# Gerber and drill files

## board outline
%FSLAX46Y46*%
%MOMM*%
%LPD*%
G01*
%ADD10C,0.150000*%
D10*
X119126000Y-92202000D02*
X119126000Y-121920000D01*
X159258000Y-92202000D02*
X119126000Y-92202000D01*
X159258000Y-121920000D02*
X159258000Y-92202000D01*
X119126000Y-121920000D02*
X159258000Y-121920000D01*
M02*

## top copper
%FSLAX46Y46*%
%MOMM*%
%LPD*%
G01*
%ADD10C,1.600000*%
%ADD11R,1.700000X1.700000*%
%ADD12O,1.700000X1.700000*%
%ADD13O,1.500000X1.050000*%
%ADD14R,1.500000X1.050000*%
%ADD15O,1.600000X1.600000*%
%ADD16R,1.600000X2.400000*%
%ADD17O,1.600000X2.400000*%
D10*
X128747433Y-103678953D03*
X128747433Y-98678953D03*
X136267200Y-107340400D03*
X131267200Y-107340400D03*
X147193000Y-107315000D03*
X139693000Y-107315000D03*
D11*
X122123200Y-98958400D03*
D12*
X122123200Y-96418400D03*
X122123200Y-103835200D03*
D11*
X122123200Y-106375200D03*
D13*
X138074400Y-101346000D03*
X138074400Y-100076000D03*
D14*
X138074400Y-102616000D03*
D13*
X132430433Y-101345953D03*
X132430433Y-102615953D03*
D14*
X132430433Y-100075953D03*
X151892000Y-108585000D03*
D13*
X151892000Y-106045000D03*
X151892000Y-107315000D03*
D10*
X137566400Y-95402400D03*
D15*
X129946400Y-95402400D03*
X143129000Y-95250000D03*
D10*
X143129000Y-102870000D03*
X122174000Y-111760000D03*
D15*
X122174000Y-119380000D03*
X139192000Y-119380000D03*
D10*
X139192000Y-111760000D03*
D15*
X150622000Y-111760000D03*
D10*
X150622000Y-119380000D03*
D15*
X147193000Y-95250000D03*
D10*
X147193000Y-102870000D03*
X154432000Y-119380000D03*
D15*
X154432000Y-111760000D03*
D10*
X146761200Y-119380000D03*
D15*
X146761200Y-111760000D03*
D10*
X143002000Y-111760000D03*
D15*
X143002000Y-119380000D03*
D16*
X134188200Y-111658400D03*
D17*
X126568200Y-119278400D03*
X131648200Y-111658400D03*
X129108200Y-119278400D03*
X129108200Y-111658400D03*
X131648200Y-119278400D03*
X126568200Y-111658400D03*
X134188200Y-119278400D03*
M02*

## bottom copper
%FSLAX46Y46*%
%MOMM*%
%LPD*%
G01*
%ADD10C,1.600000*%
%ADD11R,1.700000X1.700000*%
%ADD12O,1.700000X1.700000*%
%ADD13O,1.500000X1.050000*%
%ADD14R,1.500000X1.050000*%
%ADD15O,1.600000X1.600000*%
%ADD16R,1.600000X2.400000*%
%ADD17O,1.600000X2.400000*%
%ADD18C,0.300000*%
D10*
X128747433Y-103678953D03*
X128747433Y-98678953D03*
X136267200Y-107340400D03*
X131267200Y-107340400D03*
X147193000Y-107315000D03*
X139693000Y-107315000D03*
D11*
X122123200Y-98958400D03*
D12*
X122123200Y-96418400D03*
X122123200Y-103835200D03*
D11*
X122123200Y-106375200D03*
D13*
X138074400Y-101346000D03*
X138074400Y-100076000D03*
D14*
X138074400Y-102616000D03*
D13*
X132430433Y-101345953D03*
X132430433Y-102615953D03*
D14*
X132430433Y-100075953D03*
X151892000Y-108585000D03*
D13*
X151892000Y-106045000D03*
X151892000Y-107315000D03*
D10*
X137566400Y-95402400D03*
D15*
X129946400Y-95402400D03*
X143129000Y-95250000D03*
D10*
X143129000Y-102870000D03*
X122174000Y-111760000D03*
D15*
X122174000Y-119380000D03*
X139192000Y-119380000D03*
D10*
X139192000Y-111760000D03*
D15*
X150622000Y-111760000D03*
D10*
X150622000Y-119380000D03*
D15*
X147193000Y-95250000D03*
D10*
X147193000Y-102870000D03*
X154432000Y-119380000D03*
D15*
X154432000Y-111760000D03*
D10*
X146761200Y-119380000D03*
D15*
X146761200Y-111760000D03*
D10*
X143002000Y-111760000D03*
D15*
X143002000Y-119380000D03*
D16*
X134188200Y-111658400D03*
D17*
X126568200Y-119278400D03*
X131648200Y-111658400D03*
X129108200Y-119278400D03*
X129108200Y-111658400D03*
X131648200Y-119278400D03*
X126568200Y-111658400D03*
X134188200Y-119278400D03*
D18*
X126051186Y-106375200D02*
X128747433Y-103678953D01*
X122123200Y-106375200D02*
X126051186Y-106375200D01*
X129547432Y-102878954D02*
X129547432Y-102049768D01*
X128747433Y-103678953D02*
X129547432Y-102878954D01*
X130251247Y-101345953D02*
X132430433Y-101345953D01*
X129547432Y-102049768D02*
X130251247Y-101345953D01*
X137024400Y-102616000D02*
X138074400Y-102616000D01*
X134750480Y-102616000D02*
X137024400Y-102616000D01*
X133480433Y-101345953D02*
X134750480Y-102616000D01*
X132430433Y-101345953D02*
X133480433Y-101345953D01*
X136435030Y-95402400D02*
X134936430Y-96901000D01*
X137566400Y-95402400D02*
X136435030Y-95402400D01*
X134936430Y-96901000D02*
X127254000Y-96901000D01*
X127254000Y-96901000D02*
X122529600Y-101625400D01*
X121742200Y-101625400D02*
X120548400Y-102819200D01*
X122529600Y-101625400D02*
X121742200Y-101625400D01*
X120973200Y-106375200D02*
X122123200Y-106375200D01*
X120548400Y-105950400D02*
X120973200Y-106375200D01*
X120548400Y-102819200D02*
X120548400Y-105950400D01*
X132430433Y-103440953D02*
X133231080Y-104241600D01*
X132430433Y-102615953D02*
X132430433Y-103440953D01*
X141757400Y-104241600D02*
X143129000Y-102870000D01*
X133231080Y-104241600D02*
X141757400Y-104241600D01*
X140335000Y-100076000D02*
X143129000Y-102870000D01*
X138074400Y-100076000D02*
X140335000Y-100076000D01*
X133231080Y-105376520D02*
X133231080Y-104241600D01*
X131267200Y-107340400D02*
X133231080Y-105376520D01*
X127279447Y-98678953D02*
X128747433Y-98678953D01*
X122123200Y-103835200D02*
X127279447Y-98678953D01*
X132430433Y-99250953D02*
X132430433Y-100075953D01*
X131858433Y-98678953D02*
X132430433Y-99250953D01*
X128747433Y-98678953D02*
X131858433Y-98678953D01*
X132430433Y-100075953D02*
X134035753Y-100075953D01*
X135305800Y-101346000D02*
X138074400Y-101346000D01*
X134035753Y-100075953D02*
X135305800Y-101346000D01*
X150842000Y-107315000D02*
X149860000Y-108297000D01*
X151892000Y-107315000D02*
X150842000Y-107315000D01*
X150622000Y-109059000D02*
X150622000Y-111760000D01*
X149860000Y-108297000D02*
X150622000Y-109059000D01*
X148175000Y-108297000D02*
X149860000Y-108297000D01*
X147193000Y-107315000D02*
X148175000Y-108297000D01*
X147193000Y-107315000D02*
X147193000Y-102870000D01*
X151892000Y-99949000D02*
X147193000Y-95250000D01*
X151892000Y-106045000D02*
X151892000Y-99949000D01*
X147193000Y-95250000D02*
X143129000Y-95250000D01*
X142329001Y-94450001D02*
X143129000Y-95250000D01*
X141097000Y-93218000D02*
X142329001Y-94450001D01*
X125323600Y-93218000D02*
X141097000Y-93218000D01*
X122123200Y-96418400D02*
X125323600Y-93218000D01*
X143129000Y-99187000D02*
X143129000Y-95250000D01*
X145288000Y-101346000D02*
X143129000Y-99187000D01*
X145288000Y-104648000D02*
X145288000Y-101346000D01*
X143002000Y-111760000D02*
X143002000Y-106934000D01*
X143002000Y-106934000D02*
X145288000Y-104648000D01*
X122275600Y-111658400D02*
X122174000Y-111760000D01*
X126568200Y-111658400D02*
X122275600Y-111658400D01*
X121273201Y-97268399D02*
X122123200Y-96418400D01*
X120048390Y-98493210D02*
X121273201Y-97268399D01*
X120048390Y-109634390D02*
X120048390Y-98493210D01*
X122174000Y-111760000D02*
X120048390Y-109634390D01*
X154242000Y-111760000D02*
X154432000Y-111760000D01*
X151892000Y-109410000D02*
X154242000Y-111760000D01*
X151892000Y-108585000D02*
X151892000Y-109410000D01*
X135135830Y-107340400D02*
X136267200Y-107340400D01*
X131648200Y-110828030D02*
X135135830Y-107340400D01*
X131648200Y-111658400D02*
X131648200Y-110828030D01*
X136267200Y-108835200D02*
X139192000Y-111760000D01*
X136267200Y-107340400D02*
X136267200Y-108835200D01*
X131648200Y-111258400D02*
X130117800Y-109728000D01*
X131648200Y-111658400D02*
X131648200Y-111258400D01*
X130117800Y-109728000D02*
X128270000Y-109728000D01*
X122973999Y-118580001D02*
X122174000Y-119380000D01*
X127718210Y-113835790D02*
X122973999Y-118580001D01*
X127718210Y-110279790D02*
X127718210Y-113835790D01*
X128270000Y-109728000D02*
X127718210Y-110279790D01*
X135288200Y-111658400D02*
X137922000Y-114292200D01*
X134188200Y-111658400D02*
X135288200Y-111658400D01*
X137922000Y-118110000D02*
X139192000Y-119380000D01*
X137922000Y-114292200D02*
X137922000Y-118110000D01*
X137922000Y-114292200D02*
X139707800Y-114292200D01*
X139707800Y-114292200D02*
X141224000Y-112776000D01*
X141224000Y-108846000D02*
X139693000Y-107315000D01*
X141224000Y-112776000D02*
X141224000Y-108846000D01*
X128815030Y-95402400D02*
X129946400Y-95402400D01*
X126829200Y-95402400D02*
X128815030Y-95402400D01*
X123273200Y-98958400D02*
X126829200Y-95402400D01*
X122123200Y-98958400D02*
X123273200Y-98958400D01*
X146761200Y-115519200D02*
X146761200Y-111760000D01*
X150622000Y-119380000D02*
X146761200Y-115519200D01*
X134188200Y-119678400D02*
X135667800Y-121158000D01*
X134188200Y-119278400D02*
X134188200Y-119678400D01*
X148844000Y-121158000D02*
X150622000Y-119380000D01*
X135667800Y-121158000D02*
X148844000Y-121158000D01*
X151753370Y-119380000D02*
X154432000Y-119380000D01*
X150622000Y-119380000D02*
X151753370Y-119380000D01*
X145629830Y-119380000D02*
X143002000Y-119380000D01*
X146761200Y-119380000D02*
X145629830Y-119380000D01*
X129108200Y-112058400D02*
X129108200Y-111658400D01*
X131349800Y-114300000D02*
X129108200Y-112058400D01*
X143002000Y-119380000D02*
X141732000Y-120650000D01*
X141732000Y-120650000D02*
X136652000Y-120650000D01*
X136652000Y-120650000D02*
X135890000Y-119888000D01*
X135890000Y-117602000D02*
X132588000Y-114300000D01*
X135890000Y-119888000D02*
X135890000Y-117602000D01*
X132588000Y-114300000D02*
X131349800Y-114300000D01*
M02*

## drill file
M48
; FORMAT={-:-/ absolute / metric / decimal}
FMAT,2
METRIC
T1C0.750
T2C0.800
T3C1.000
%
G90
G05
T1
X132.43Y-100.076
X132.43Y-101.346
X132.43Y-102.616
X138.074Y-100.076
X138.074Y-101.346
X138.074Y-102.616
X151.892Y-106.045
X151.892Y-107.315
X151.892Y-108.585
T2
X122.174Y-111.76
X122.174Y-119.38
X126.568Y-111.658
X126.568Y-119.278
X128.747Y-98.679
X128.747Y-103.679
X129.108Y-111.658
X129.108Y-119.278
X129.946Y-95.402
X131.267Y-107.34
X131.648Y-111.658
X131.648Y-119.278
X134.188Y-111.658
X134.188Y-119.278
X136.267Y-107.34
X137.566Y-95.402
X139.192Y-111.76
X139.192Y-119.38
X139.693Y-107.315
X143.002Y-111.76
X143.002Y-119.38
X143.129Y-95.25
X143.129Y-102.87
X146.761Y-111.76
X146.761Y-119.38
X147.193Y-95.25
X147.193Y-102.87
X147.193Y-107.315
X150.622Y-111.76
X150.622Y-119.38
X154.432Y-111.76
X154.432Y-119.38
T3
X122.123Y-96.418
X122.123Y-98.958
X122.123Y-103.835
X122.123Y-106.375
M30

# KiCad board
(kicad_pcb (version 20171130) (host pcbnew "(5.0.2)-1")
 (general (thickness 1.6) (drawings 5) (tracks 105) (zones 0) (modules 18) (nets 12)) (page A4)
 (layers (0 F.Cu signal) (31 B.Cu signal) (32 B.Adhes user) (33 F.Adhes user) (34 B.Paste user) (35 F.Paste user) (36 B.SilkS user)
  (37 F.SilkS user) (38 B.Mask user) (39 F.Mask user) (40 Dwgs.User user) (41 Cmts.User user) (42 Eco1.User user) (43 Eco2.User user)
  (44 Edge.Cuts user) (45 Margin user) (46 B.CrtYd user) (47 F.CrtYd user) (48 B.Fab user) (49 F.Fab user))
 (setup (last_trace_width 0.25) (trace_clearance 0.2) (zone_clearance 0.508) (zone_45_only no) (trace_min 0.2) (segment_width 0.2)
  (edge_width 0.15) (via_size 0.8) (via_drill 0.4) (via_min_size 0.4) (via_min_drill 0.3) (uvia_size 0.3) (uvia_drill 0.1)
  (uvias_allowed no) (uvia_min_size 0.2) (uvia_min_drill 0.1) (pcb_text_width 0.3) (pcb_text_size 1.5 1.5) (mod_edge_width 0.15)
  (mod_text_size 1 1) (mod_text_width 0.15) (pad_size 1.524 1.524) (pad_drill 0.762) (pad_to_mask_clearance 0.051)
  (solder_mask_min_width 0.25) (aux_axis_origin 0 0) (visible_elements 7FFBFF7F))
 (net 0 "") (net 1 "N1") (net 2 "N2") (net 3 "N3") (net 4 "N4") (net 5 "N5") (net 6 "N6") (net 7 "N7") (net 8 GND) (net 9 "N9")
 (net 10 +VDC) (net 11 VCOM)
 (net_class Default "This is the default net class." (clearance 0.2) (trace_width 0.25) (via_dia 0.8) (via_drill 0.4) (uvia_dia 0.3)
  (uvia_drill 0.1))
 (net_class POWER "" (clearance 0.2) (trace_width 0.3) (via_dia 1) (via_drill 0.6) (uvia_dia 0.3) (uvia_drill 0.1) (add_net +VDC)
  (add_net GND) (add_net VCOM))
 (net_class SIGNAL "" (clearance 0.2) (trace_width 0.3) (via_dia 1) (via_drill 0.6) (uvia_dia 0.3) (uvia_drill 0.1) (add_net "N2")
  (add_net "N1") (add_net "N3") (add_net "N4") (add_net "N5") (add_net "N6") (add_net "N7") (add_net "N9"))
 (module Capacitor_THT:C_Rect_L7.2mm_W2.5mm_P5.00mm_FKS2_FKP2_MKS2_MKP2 (layer F.Cu) (at 128.747433 98.678953 270)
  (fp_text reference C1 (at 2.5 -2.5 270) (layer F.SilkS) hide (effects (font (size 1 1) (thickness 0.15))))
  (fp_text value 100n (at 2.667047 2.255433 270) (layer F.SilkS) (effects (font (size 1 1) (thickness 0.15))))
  (pad 2 thru_hole circle (at 5 0 270) (size 1.6 1.6) (drill 0.8) (layers *.Cu *.Mask) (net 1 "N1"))
  (pad 1 thru_hole circle (at 0 0 270) (size 1.6 1.6) (drill 0.8) (layers *.Cu *.Mask) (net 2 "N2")))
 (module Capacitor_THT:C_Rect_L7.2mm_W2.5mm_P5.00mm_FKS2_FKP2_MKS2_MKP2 (layer F.Cu) (at 136.2672 107.3404 180)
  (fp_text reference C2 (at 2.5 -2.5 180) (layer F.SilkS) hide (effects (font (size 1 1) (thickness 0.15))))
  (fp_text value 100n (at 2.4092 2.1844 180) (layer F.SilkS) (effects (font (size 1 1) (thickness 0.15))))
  (pad 1 thru_hole circle (at 0 0 180) (size 1.6 1.6) (drill 0.8) (layers *.Cu *.Mask) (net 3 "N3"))
  (pad 2 thru_hole circle (at 5 0 180) (size 1.6 1.6) (drill 0.8) (layers *.Cu *.Mask) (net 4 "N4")))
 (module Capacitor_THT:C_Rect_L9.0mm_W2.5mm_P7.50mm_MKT (layer F.Cu) (at 147.193 107.315 180)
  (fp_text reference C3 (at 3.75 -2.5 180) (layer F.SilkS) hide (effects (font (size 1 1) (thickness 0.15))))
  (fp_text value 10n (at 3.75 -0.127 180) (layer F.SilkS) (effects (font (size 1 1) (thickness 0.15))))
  (pad 1 thru_hole circle (at 0 0 180) (size 1.6 1.6) (drill 0.8) (layers *.Cu *.Mask) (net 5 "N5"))
  (pad 2 thru_hole circle (at 7.5 0 180) (size 1.6 1.6) (drill 0.8) (layers *.Cu *.Mask) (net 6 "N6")))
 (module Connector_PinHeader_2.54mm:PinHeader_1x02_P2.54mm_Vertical (layer F.Cu) (at 122.1232 98.9584 180)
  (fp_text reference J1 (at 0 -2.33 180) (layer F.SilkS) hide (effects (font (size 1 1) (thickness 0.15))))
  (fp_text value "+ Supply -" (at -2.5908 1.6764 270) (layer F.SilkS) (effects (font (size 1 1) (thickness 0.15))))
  (pad 1 thru_hole rect (at 0 0 180) (size 1.7 1.7) (drill 1) (layers *.Cu *.Mask) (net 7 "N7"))
  (pad 2 thru_hole oval (at 0 2.54 180) (size 1.7 1.7) (drill 1) (layers *.Cu *.Mask) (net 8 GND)))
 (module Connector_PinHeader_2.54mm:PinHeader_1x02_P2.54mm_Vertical (layer F.Cu) (at 122.1232 106.3752 180)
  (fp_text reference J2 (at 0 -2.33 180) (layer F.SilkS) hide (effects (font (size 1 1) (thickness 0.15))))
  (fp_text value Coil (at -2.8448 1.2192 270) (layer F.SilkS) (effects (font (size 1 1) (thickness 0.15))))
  (pad 2 thru_hole oval (at 0 2.54 180) (size 1.7 1.7) (drill 1) (layers *.Cu *.Mask) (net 2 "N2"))
  (pad 1 thru_hole rect (at 0 0 180) (size 1.7 1.7) (drill 1) (layers *.Cu *.Mask) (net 1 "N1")))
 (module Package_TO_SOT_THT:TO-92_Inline (layer F.Cu) (at 138.0744 102.616 90)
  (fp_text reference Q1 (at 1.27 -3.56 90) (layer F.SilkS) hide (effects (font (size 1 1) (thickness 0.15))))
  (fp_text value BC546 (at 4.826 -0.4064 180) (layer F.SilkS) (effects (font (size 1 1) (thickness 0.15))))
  (pad 2 thru_hole oval (at 1.27 0 90) (size 1.05 1.5) (drill 0.75) (layers *.Cu *.Mask) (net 2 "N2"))
  (pad 3 thru_hole oval (at 2.54 0 90) (size 1.05 1.5) (drill 0.75) (layers *.Cu *.Mask) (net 4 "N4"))
  (pad 1 thru_hole rect (at 0 0 90) (size 1.05 1.5) (drill 0.75) (layers *.Cu *.Mask) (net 1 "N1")))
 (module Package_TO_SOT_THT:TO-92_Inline (layer F.Cu) (at 132.430433 100.075953 270)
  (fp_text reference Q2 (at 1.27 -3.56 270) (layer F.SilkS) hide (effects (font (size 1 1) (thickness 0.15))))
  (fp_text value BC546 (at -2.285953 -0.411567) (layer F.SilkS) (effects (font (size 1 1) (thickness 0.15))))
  (pad 2 thru_hole oval (at 1.27 0 270) (size 1.05 1.5) (drill 0.75) (layers *.Cu *.Mask) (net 1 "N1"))
  (pad 3 thru_hole oval (at 2.54 0 270) (size 1.05 1.5) (drill 0.75) (layers *.Cu *.Mask) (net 4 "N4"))
  (pad 1 thru_hole rect (at 0 0 270) (size 1.05 1.5) (drill 0.75) (layers *.Cu *.Mask) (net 2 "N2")))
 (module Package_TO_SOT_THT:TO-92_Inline (layer F.Cu) (at 151.892 108.585 90)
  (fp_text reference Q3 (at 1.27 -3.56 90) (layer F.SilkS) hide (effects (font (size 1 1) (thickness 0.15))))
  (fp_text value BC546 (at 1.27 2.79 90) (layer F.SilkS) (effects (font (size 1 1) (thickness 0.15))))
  (pad 1 thru_hole rect (at 0 0 90) (size 1.05 1.5) (drill 0.75) (layers *.Cu *.Mask) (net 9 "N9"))
  (pad 3 thru_hole oval (at 2.54 0 90) (size 1.05 1.5) (drill 0.75) (layers *.Cu *.Mask) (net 8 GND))
  (pad 2 thru_hole oval (at 1.27 0 90) (size 1.05 1.5) (drill 0.75) (layers *.Cu *.Mask) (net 5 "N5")))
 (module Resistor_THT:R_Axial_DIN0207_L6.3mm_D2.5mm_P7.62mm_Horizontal (layer F.Cu) (at 137.5664 95.4024 180)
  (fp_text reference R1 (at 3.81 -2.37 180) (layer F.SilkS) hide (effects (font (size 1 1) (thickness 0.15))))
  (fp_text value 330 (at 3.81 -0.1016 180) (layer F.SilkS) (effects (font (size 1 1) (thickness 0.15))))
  (pad 1 thru_hole circle (at 0 0 180) (size 1.6 1.6) (drill 0.8) (layers *.Cu *.Mask) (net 1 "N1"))
  (pad 2 thru_hole oval (at 7.62 0 180) (size 1.6 1.6) (drill 0.8) (layers *.Cu *.Mask) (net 7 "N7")))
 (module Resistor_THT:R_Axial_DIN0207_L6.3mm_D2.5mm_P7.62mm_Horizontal (layer F.Cu) (at 143.129 102.87 90)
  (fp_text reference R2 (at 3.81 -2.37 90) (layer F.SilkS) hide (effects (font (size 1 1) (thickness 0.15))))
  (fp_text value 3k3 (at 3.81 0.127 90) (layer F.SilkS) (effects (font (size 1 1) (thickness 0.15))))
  (pad 2 thru_hole oval (at 7.62 0 90) (size 1.6 1.6) (drill 0.8) (layers *.Cu *.Mask) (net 8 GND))
  (pad 1 thru_hole circle (at 0 0 90) (size 1.6 1.6) (drill 0.8) (layers *.Cu *.Mask) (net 4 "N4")))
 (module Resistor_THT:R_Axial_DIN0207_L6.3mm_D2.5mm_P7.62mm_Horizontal (layer F.Cu) (at 122.174 111.76 270)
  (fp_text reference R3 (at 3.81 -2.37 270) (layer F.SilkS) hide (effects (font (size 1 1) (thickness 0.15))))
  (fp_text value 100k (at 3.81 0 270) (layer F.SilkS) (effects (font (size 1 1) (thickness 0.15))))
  (pad 1 thru_hole circle (at 0 0 270) (size 1.6 1.6) (drill 0.8) (layers *.Cu *.Mask) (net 8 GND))
  (pad 2 thru_hole oval (at 7.62 0 270) (size 1.6 1.6) (drill 0.8) (layers *.Cu *.Mask) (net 3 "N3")))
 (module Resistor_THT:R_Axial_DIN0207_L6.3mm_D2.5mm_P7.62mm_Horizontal (layer F.Cu) (at 139.192 111.76 270)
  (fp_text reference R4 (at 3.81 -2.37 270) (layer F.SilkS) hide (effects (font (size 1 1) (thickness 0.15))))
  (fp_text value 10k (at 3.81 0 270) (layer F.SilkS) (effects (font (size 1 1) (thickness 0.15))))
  (pad 2 thru_hole oval (at 7.62 0 270) (size 1.6 1.6) (drill 0.8) (layers *.Cu *.Mask) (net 6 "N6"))
  (pad 1 thru_hole circle (at 0 0 270) (size 1.6 1.6) (drill 0.8) (layers *.Cu *.Mask) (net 3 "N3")))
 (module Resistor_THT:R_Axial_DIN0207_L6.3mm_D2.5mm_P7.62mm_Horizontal (layer F.Cu) (at 150.622 119.38 90)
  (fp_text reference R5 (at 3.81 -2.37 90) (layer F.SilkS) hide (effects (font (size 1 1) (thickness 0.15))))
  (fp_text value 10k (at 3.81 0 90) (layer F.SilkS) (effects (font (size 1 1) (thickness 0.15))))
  (pad 2 thru_hole oval (at 7.62 0 90) (size 1.6 1.6) (drill 0.8) (layers *.Cu *.Mask) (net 5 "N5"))
  (pad 1 thru_hole circle (at 0 0 90) (size 1.6 1.6) (drill 0.8) (layers *.Cu *.Mask) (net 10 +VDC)))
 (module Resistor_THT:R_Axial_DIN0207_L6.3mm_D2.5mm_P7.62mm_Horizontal (layer F.Cu) (at 147.193 102.87 90)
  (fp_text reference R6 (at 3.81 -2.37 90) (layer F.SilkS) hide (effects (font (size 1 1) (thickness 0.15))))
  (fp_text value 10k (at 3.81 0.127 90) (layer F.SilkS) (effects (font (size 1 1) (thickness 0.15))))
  (pad 2 thru_hole oval (at 7.62 0 90) (size 1.6 1.6) (drill 0.8) (layers *.Cu *.Mask) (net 8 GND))
  (pad 1 thru_hole circle (at 0 0 90) (size 1.6 1.6) (drill 0.8) (layers *.Cu *.Mask) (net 5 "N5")))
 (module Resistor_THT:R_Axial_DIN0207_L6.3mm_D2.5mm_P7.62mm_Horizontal (layer F.Cu) (at 154.432 119.38 90)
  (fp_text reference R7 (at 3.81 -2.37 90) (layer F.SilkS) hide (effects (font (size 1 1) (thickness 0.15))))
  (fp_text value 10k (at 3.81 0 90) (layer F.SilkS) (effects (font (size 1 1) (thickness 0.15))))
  (pad 1 thru_hole circle (at 0 0 90) (size 1.6 1.6) (drill 0.8) (layers *.Cu *.Mask) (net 10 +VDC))
  (pad 2 thru_hole oval (at 7.62 0 90) (size 1.6 1.6) (drill 0.8) (layers *.Cu *.Mask) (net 9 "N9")))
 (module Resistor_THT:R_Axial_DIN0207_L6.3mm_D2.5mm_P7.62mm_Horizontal (layer F.Cu) (at 146.7612 119.38 90)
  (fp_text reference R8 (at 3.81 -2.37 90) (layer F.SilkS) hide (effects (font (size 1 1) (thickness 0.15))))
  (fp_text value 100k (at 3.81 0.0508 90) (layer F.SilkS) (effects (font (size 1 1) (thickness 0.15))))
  (pad 1 thru_hole circle (at 0 0 90) (size 1.6 1.6) (drill 0.8) (layers *.Cu *.Mask) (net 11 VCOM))
  (pad 2 thru_hole oval (at 7.62 0 90) (size 1.6 1.6) (drill 0.8) (layers *.Cu *.Mask) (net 10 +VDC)))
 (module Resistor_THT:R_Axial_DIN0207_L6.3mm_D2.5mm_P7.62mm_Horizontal (layer F.Cu) (at 143.002 111.76 270)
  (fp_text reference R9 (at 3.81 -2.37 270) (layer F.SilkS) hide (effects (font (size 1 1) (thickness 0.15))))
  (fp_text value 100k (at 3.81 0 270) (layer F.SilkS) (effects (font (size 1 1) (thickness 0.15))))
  (pad 1 thru_hole circle (at 0 0 270) (size 1.6 1.6) (drill 0.8) (layers *.Cu *.Mask) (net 8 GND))
  (pad 2 thru_hole oval (at 7.62 0 270) (size 1.6 1.6) (drill 0.8) (layers *.Cu *.Mask) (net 11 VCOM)))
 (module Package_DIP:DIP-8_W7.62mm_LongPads (layer F.Cu) (at 134.1882 111.6584 270)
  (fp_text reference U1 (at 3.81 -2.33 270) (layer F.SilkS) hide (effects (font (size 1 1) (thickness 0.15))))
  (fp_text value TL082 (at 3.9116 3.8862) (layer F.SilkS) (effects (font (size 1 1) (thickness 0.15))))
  (pad 1 thru_hole rect (at 0 0 270) (size 2.4 1.6) (drill 0.8) (layers *.Cu *.Mask) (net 6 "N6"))
  (pad 5 thru_hole oval (at 7.62 7.62 270) (size 2.4 1.6) (drill 0.8) (layers *.Cu *.Mask))
  (pad 2 thru_hole oval (at 0 2.54 270) (size 2.4 1.6) (drill 0.8) (layers *.Cu *.Mask) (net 3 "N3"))
  (pad 6 thru_hole oval (at 7.62 5.08 270) (size 2.4 1.6) (drill 0.8) (layers *.Cu *.Mask))
  (pad 3 thru_hole oval (at 0 5.08 270) (size 2.4 1.6) (drill 0.8) (layers *.Cu *.Mask) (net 11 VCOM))
  (pad 7 thru_hole oval (at 7.62 2.54 270) (size 2.4 1.6) (drill 0.8) (layers *.Cu *.Mask))
  (pad 4 thru_hole oval (at 0 7.62 270) (size 2.4 1.6) (drill 0.8) (layers *.Cu *.Mask) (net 8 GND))
  (pad 8 thru_hole oval (at 7.62 0 270) (size 2.4 1.6) (drill 0.8) (layers *.Cu *.Mask) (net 10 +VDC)))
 (gr_line (start 119.126 92.202) (end 119.126 121.92) (layer Edge.Cuts) (width 0.15))
 (gr_line (start 159.258 92.202) (end 119.126 92.202) (layer Edge.Cuts) (width 0.15))
 (gr_line (start 159.258 121.92) (end 159.258 92.202) (layer Edge.Cuts) (width 0.15))
 (gr_line (start 119.126 121.92) (end 159.258 121.92) (layer Edge.Cuts) (width 0.15))
 (segment (start 126.051186 106.3752) (end 128.747433 103.678953) (width 0.3) (layer B.Cu) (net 1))
 (segment (start 122.1232 106.3752) (end 126.051186 106.3752) (width 0.3) (layer B.Cu) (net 1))
 (segment (start 129.547432 102.878954) (end 129.547432 102.049768) (width 0.3) (layer B.Cu) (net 1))
 (segment (start 128.747433 103.678953) (end 129.547432 102.878954) (width 0.3) (layer B.Cu) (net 1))
 (segment (start 130.251247 101.345953) (end 132.430433 101.345953) (width 0.3) (layer B.Cu) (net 1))
 (segment (start 129.547432 102.049768) (end 130.251247 101.345953) (width 0.3) (layer B.Cu) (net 1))
 (segment (start 137.0244 102.616) (end 138.0744 102.616) (width 0.3) (layer B.Cu) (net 1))
 (segment (start 134.75048 102.616) (end 137.0244 102.616) (width 0.3) (layer B.Cu) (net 1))
 (segment (start 133.480433 101.345953) (end 134.75048 102.616) (width 0.3) (layer B.Cu) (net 1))
 (segment (start 132.430433 101.345953) (end 133.480433 101.345953) (width 0.3) (layer B.Cu) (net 1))
 (segment (start 136.43503 95.4024) (end 134.93643 96.901) (width 0.3) (layer B.Cu) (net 1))
 (segment (start 137.5664 95.4024) (end 136.43503 95.4024) (width 0.3) (layer B.Cu) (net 1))
 (segment (start 134.93643 96.901) (end 127.254 96.901) (width 0.3) (layer B.Cu) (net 1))
 (segment (start 127.254 96.901) (end 122.5296 101.6254) (width 0.3) (layer B.Cu) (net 1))
 (segment (start 121.7422 101.6254) (end 120.5484 102.8192) (width 0.3) (layer B.Cu) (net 1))
 (segment (start 122.5296 101.6254) (end 121.7422 101.6254) (width 0.3) (layer B.Cu) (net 1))
 (segment (start 120.9732 106.3752) (end 122.1232 106.3752) (width 0.3) (layer B.Cu) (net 1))
 (segment (start 120.5484 105.9504) (end 120.9732 106.3752) (width 0.3) (layer B.Cu) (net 1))
 (segment (start 120.5484 102.8192) (end 120.5484 105.9504) (width 0.3) (layer B.Cu) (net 1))
 (segment (start 132.430433 103.440953) (end 133.23108 104.2416) (width 0.3) (layer B.Cu) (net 4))
 (segment (start 132.430433 102.615953) (end 132.430433 103.440953) (width 0.3) (layer B.Cu) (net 4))
 (segment (start 141.7574 104.2416) (end 143.129 102.87) (width 0.3) (layer B.Cu) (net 4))
 (segment (start 133.23108 104.2416) (end 141.7574 104.2416) (width 0.3) (layer B.Cu) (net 4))
 (segment (start 140.335 100.076) (end 143.129 102.87) (width 0.3) (layer B.Cu) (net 4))
 (segment (start 138.0744 100.076) (end 140.335 100.076) (width 0.3) (layer B.Cu) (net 4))
 (segment (start 133.23108 105.37652) (end 133.23108 104.2416) (width 0.3) (layer B.Cu) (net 4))
 (segment (start 131.2672 107.3404) (end 133.23108 105.37652) (width 0.3) (layer B.Cu) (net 4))
 (segment (start 127.279447 98.678953) (end 128.747433 98.678953) (width 0.3) (layer B.Cu) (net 2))
 (segment (start 122.1232 103.8352) (end 127.279447 98.678953) (width 0.3) (layer B.Cu) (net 2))
 (segment (start 132.430433 99.250953) (end 132.430433 100.075953) (width 0.3) (layer B.Cu) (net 2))
 (segment (start 131.858433 98.678953) (end 132.430433 99.250953) (width 0.3) (layer B.Cu) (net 2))
 (segment (start 128.747433 98.678953) (end 131.858433 98.678953) (width 0.3) (layer B.Cu) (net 2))
 (segment (start 132.430433 100.075953) (end 134.035753 100.075953) (width 0.3) (layer B.Cu) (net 2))
 (segment (start 135.3058 101.346) (end 138.0744 101.346) (width 0.3) (layer B.Cu) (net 2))
 (segment (start 134.035753 100.075953) (end 135.3058 101.346) (width 0.3) (layer B.Cu) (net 2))
 (segment (start 150.842 107.315) (end 149.86 108.297) (width 0.3) (layer B.Cu) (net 5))
 (segment (start 151.892 107.315) (end 150.842 107.315) (width 0.3) (layer B.Cu) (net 5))
 (segment (start 150.622 109.059) (end 150.622 111.76) (width 0.3) (layer B.Cu) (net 5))
 (segment (start 149.86 108.297) (end 150.622 109.059) (width 0.3) (layer B.Cu) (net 5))
 (segment (start 148.175 108.297) (end 149.86 108.297) (width 0.3) (layer B.Cu) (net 5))
 (segment (start 147.193 107.315) (end 148.175 108.297) (width 0.3) (layer B.Cu) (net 5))
 (segment (start 147.193 107.315) (end 147.193 102.87) (width 0.3) (layer B.Cu) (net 5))
 (segment (start 151.892 99.949) (end 147.193 95.25) (width 0.3) (layer B.Cu) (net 8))
 (segment (start 151.892 106.045) (end 151.892 99.949) (width 0.3) (layer B.Cu) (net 8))
 (segment (start 147.193 95.25) (end 143.129 95.25) (width 0.3) (layer B.Cu) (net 8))
 (segment (start 142.329001 94.450001) (end 143.129 95.25) (width 0.3) (layer B.Cu) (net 8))
 (segment (start 141.097 93.218) (end 142.329001 94.450001) (width 0.3) (layer B.Cu) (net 8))
 (segment (start 125.3236 93.218) (end 141.097 93.218) (width 0.3) (layer B.Cu) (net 8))
 (segment (start 122.1232 96.4184) (end 125.3236 93.218) (width 0.3) (layer B.Cu) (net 8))
 (segment (start 143.129 99.187) (end 143.129 95.25) (width 0.3) (layer B.Cu) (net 8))
 (segment (start 145.288 101.346) (end 143.129 99.187) (width 0.3) (layer B.Cu) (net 8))
 (segment (start 145.288 104.648) (end 145.288 101.346) (width 0.3) (layer B.Cu) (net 8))
 (segment (start 143.002 111.76) (end 143.002 106.934) (width 0.3) (layer B.Cu) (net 8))
 (segment (start 143.002 106.934) (end 145.288 104.648) (width 0.3) (layer B.Cu) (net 8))
 (segment (start 122.2756 111.6584) (end 122.174 111.76) (width 0.3) (layer B.Cu) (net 8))
 (segment (start 126.5682 111.6584) (end 122.2756 111.6584) (width 0.3) (layer B.Cu) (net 8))
 (segment (start 121.273201 97.268399) (end 122.1232 96.4184) (width 0.3) (layer B.Cu) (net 8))
 (segment (start 120.04839 98.49321) (end 121.273201 97.268399) (width 0.3) (layer B.Cu) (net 8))
 (segment (start 120.04839 109.63439) (end 120.04839 98.49321) (width 0.3) (layer B.Cu) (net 8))
 (segment (start 122.174 111.76) (end 120.04839 109.63439) (width 0.3) (layer B.Cu) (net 8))
 (segment (start 154.242 111.76) (end 154.432 111.76) (width 0.3) (layer B.Cu) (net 9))
 (segment (start 151.892 109.41) (end 154.242 111.76) (width 0.3) (layer B.Cu) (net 9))
 (segment (start 151.892 108.585) (end 151.892 109.41) (width 0.3) (layer B.Cu) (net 9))
 (segment (start 135.13583 107.3404) (end 136.2672 107.3404) (width 0.3) (layer B.Cu) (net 3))
 (segment (start 131.6482 110.82803) (end 135.13583 107.3404) (width 0.3) (layer B.Cu) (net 3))
 (segment (start 131.6482 111.6584) (end 131.6482 110.82803) (width 0.3) (layer B.Cu) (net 3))
 (segment (start 136.2672 108.8352) (end 139.192 111.76) (width 0.3) (layer B.Cu) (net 3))
 (segment (start 136.2672 107.3404) (end 136.2672 108.8352) (width 0.3) (layer B.Cu) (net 3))
 (segment (start 131.6482 111.2584) (end 130.1178 109.728) (width 0.3) (layer B.Cu) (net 3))
 (segment (start 131.6482 111.6584) (end 131.6482 111.2584) (width 0.3) (layer B.Cu) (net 3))
 (segment (start 130.1178 109.728) (end 128.27 109.728) (width 0.3) (layer B.Cu) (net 3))
 (segment (start 122.973999 118.580001) (end 122.174 119.38) (width 0.3) (layer B.Cu) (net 3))
 (segment (start 127.71821 113.83579) (end 122.973999 118.580001) (width 0.3) (layer B.Cu) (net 3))
 (segment (start 127.71821 110.27979) (end 127.71821 113.83579) (width 0.3) (layer B.Cu) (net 3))
 (segment (start 128.27 109.728) (end 127.71821 110.27979) (width 0.3) (layer B.Cu) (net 3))
 (segment (start 135.2882 111.6584) (end 137.922 114.2922) (width 0.3) (layer B.Cu) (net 6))
 (segment (start 134.1882 111.6584) (end 135.2882 111.6584) (width 0.3) (layer B.Cu) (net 6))
 (segment (start 137.922 118.11) (end 139.192 119.38) (width 0.3) (layer B.Cu) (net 6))
 (segment (start 137.922 114.2922) (end 137.922 118.11) (width 0.3) (layer B.Cu) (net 6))
 (segment (start 137.922 114.2922) (end 139.7078 114.2922) (width 0.3) (layer B.Cu) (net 6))
 (segment (start 139.7078 114.2922) (end 141.224 112.776) (width 0.3) (layer B.Cu) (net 6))
 (segment (start 141.224 108.846) (end 139.693 107.315) (width 0.3) (layer B.Cu) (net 6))
 (segment (start 141.224 112.776) (end 141.224 108.846) (width 0.3) (layer B.Cu) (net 6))
 (segment (start 128.81503 95.4024) (end 129.9464 95.4024) (width 0.3) (layer B.Cu) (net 7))
 (segment (start 126.8292 95.4024) (end 128.81503 95.4024) (width 0.3) (layer B.Cu) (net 7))
 (segment (start 123.2732 98.9584) (end 126.8292 95.4024) (width 0.3) (layer B.Cu) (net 7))
 (segment (start 122.1232 98.9584) (end 123.2732 98.9584) (width 0.3) (layer B.Cu) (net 7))
 (segment (start 146.7612 115.5192) (end 146.7612 111.76) (width 0.3) (layer B.Cu) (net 10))
 (segment (start 150.622 119.38) (end 146.7612 115.5192) (width 0.3) (layer B.Cu) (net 10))
 (segment (start 134.1882 119.6784) (end 135.6678 121.158) (width 0.3) (layer B.Cu) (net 10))
 (segment (start 134.1882 119.2784) (end 134.1882 119.6784) (width 0.3) (layer B.Cu) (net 10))
 (segment (start 148.844 121.158) (end 150.622 119.38) (width 0.3) (layer B.Cu) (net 10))
 (segment (start 135.6678 121.158) (end 148.844 121.158) (width 0.3) (layer B.Cu) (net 10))
 (segment (start 151.75337 119.38) (end 154.432 119.38) (width 0.3) (layer B.Cu) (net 10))
 (segment (start 150.622 119.38) (end 151.75337 119.38) (width 0.3) (layer B.Cu) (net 10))
 (segment (start 145.62983 119.38) (end 143.002 119.38) (width 0.3) (layer B.Cu) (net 11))
 (segment (start 146.7612 119.38) (end 145.62983 119.38) (width 0.3) (layer B.Cu) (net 11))
 (segment (start 129.1082 112.0584) (end 129.1082 111.6584) (width 0.3) (layer B.Cu) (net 11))
 (segment (start 131.3498 114.3) (end 129.1082 112.0584) (width 0.3) (layer B.Cu) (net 11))
 (segment (start 143.002 119.38) (end 141.732 120.65) (width 0.3) (layer B.Cu) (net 11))
 (segment (start 141.732 120.65) (end 136.652 120.65) (width 0.3) (layer B.Cu) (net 11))
 (segment (start 136.652 120.65) (end 135.89 119.888) (width 0.3) (layer B.Cu) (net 11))
 (segment (start 135.89 117.602) (end 132.588 114.3) (width 0.3) (layer B.Cu) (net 11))
 (segment (start 135.89 119.888) (end 135.89 117.602) (width 0.3) (layer B.Cu) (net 11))
 (segment (start 132.588 114.3) (end 131.3498 114.3) (width 0.3) (layer B.Cu) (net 11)))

